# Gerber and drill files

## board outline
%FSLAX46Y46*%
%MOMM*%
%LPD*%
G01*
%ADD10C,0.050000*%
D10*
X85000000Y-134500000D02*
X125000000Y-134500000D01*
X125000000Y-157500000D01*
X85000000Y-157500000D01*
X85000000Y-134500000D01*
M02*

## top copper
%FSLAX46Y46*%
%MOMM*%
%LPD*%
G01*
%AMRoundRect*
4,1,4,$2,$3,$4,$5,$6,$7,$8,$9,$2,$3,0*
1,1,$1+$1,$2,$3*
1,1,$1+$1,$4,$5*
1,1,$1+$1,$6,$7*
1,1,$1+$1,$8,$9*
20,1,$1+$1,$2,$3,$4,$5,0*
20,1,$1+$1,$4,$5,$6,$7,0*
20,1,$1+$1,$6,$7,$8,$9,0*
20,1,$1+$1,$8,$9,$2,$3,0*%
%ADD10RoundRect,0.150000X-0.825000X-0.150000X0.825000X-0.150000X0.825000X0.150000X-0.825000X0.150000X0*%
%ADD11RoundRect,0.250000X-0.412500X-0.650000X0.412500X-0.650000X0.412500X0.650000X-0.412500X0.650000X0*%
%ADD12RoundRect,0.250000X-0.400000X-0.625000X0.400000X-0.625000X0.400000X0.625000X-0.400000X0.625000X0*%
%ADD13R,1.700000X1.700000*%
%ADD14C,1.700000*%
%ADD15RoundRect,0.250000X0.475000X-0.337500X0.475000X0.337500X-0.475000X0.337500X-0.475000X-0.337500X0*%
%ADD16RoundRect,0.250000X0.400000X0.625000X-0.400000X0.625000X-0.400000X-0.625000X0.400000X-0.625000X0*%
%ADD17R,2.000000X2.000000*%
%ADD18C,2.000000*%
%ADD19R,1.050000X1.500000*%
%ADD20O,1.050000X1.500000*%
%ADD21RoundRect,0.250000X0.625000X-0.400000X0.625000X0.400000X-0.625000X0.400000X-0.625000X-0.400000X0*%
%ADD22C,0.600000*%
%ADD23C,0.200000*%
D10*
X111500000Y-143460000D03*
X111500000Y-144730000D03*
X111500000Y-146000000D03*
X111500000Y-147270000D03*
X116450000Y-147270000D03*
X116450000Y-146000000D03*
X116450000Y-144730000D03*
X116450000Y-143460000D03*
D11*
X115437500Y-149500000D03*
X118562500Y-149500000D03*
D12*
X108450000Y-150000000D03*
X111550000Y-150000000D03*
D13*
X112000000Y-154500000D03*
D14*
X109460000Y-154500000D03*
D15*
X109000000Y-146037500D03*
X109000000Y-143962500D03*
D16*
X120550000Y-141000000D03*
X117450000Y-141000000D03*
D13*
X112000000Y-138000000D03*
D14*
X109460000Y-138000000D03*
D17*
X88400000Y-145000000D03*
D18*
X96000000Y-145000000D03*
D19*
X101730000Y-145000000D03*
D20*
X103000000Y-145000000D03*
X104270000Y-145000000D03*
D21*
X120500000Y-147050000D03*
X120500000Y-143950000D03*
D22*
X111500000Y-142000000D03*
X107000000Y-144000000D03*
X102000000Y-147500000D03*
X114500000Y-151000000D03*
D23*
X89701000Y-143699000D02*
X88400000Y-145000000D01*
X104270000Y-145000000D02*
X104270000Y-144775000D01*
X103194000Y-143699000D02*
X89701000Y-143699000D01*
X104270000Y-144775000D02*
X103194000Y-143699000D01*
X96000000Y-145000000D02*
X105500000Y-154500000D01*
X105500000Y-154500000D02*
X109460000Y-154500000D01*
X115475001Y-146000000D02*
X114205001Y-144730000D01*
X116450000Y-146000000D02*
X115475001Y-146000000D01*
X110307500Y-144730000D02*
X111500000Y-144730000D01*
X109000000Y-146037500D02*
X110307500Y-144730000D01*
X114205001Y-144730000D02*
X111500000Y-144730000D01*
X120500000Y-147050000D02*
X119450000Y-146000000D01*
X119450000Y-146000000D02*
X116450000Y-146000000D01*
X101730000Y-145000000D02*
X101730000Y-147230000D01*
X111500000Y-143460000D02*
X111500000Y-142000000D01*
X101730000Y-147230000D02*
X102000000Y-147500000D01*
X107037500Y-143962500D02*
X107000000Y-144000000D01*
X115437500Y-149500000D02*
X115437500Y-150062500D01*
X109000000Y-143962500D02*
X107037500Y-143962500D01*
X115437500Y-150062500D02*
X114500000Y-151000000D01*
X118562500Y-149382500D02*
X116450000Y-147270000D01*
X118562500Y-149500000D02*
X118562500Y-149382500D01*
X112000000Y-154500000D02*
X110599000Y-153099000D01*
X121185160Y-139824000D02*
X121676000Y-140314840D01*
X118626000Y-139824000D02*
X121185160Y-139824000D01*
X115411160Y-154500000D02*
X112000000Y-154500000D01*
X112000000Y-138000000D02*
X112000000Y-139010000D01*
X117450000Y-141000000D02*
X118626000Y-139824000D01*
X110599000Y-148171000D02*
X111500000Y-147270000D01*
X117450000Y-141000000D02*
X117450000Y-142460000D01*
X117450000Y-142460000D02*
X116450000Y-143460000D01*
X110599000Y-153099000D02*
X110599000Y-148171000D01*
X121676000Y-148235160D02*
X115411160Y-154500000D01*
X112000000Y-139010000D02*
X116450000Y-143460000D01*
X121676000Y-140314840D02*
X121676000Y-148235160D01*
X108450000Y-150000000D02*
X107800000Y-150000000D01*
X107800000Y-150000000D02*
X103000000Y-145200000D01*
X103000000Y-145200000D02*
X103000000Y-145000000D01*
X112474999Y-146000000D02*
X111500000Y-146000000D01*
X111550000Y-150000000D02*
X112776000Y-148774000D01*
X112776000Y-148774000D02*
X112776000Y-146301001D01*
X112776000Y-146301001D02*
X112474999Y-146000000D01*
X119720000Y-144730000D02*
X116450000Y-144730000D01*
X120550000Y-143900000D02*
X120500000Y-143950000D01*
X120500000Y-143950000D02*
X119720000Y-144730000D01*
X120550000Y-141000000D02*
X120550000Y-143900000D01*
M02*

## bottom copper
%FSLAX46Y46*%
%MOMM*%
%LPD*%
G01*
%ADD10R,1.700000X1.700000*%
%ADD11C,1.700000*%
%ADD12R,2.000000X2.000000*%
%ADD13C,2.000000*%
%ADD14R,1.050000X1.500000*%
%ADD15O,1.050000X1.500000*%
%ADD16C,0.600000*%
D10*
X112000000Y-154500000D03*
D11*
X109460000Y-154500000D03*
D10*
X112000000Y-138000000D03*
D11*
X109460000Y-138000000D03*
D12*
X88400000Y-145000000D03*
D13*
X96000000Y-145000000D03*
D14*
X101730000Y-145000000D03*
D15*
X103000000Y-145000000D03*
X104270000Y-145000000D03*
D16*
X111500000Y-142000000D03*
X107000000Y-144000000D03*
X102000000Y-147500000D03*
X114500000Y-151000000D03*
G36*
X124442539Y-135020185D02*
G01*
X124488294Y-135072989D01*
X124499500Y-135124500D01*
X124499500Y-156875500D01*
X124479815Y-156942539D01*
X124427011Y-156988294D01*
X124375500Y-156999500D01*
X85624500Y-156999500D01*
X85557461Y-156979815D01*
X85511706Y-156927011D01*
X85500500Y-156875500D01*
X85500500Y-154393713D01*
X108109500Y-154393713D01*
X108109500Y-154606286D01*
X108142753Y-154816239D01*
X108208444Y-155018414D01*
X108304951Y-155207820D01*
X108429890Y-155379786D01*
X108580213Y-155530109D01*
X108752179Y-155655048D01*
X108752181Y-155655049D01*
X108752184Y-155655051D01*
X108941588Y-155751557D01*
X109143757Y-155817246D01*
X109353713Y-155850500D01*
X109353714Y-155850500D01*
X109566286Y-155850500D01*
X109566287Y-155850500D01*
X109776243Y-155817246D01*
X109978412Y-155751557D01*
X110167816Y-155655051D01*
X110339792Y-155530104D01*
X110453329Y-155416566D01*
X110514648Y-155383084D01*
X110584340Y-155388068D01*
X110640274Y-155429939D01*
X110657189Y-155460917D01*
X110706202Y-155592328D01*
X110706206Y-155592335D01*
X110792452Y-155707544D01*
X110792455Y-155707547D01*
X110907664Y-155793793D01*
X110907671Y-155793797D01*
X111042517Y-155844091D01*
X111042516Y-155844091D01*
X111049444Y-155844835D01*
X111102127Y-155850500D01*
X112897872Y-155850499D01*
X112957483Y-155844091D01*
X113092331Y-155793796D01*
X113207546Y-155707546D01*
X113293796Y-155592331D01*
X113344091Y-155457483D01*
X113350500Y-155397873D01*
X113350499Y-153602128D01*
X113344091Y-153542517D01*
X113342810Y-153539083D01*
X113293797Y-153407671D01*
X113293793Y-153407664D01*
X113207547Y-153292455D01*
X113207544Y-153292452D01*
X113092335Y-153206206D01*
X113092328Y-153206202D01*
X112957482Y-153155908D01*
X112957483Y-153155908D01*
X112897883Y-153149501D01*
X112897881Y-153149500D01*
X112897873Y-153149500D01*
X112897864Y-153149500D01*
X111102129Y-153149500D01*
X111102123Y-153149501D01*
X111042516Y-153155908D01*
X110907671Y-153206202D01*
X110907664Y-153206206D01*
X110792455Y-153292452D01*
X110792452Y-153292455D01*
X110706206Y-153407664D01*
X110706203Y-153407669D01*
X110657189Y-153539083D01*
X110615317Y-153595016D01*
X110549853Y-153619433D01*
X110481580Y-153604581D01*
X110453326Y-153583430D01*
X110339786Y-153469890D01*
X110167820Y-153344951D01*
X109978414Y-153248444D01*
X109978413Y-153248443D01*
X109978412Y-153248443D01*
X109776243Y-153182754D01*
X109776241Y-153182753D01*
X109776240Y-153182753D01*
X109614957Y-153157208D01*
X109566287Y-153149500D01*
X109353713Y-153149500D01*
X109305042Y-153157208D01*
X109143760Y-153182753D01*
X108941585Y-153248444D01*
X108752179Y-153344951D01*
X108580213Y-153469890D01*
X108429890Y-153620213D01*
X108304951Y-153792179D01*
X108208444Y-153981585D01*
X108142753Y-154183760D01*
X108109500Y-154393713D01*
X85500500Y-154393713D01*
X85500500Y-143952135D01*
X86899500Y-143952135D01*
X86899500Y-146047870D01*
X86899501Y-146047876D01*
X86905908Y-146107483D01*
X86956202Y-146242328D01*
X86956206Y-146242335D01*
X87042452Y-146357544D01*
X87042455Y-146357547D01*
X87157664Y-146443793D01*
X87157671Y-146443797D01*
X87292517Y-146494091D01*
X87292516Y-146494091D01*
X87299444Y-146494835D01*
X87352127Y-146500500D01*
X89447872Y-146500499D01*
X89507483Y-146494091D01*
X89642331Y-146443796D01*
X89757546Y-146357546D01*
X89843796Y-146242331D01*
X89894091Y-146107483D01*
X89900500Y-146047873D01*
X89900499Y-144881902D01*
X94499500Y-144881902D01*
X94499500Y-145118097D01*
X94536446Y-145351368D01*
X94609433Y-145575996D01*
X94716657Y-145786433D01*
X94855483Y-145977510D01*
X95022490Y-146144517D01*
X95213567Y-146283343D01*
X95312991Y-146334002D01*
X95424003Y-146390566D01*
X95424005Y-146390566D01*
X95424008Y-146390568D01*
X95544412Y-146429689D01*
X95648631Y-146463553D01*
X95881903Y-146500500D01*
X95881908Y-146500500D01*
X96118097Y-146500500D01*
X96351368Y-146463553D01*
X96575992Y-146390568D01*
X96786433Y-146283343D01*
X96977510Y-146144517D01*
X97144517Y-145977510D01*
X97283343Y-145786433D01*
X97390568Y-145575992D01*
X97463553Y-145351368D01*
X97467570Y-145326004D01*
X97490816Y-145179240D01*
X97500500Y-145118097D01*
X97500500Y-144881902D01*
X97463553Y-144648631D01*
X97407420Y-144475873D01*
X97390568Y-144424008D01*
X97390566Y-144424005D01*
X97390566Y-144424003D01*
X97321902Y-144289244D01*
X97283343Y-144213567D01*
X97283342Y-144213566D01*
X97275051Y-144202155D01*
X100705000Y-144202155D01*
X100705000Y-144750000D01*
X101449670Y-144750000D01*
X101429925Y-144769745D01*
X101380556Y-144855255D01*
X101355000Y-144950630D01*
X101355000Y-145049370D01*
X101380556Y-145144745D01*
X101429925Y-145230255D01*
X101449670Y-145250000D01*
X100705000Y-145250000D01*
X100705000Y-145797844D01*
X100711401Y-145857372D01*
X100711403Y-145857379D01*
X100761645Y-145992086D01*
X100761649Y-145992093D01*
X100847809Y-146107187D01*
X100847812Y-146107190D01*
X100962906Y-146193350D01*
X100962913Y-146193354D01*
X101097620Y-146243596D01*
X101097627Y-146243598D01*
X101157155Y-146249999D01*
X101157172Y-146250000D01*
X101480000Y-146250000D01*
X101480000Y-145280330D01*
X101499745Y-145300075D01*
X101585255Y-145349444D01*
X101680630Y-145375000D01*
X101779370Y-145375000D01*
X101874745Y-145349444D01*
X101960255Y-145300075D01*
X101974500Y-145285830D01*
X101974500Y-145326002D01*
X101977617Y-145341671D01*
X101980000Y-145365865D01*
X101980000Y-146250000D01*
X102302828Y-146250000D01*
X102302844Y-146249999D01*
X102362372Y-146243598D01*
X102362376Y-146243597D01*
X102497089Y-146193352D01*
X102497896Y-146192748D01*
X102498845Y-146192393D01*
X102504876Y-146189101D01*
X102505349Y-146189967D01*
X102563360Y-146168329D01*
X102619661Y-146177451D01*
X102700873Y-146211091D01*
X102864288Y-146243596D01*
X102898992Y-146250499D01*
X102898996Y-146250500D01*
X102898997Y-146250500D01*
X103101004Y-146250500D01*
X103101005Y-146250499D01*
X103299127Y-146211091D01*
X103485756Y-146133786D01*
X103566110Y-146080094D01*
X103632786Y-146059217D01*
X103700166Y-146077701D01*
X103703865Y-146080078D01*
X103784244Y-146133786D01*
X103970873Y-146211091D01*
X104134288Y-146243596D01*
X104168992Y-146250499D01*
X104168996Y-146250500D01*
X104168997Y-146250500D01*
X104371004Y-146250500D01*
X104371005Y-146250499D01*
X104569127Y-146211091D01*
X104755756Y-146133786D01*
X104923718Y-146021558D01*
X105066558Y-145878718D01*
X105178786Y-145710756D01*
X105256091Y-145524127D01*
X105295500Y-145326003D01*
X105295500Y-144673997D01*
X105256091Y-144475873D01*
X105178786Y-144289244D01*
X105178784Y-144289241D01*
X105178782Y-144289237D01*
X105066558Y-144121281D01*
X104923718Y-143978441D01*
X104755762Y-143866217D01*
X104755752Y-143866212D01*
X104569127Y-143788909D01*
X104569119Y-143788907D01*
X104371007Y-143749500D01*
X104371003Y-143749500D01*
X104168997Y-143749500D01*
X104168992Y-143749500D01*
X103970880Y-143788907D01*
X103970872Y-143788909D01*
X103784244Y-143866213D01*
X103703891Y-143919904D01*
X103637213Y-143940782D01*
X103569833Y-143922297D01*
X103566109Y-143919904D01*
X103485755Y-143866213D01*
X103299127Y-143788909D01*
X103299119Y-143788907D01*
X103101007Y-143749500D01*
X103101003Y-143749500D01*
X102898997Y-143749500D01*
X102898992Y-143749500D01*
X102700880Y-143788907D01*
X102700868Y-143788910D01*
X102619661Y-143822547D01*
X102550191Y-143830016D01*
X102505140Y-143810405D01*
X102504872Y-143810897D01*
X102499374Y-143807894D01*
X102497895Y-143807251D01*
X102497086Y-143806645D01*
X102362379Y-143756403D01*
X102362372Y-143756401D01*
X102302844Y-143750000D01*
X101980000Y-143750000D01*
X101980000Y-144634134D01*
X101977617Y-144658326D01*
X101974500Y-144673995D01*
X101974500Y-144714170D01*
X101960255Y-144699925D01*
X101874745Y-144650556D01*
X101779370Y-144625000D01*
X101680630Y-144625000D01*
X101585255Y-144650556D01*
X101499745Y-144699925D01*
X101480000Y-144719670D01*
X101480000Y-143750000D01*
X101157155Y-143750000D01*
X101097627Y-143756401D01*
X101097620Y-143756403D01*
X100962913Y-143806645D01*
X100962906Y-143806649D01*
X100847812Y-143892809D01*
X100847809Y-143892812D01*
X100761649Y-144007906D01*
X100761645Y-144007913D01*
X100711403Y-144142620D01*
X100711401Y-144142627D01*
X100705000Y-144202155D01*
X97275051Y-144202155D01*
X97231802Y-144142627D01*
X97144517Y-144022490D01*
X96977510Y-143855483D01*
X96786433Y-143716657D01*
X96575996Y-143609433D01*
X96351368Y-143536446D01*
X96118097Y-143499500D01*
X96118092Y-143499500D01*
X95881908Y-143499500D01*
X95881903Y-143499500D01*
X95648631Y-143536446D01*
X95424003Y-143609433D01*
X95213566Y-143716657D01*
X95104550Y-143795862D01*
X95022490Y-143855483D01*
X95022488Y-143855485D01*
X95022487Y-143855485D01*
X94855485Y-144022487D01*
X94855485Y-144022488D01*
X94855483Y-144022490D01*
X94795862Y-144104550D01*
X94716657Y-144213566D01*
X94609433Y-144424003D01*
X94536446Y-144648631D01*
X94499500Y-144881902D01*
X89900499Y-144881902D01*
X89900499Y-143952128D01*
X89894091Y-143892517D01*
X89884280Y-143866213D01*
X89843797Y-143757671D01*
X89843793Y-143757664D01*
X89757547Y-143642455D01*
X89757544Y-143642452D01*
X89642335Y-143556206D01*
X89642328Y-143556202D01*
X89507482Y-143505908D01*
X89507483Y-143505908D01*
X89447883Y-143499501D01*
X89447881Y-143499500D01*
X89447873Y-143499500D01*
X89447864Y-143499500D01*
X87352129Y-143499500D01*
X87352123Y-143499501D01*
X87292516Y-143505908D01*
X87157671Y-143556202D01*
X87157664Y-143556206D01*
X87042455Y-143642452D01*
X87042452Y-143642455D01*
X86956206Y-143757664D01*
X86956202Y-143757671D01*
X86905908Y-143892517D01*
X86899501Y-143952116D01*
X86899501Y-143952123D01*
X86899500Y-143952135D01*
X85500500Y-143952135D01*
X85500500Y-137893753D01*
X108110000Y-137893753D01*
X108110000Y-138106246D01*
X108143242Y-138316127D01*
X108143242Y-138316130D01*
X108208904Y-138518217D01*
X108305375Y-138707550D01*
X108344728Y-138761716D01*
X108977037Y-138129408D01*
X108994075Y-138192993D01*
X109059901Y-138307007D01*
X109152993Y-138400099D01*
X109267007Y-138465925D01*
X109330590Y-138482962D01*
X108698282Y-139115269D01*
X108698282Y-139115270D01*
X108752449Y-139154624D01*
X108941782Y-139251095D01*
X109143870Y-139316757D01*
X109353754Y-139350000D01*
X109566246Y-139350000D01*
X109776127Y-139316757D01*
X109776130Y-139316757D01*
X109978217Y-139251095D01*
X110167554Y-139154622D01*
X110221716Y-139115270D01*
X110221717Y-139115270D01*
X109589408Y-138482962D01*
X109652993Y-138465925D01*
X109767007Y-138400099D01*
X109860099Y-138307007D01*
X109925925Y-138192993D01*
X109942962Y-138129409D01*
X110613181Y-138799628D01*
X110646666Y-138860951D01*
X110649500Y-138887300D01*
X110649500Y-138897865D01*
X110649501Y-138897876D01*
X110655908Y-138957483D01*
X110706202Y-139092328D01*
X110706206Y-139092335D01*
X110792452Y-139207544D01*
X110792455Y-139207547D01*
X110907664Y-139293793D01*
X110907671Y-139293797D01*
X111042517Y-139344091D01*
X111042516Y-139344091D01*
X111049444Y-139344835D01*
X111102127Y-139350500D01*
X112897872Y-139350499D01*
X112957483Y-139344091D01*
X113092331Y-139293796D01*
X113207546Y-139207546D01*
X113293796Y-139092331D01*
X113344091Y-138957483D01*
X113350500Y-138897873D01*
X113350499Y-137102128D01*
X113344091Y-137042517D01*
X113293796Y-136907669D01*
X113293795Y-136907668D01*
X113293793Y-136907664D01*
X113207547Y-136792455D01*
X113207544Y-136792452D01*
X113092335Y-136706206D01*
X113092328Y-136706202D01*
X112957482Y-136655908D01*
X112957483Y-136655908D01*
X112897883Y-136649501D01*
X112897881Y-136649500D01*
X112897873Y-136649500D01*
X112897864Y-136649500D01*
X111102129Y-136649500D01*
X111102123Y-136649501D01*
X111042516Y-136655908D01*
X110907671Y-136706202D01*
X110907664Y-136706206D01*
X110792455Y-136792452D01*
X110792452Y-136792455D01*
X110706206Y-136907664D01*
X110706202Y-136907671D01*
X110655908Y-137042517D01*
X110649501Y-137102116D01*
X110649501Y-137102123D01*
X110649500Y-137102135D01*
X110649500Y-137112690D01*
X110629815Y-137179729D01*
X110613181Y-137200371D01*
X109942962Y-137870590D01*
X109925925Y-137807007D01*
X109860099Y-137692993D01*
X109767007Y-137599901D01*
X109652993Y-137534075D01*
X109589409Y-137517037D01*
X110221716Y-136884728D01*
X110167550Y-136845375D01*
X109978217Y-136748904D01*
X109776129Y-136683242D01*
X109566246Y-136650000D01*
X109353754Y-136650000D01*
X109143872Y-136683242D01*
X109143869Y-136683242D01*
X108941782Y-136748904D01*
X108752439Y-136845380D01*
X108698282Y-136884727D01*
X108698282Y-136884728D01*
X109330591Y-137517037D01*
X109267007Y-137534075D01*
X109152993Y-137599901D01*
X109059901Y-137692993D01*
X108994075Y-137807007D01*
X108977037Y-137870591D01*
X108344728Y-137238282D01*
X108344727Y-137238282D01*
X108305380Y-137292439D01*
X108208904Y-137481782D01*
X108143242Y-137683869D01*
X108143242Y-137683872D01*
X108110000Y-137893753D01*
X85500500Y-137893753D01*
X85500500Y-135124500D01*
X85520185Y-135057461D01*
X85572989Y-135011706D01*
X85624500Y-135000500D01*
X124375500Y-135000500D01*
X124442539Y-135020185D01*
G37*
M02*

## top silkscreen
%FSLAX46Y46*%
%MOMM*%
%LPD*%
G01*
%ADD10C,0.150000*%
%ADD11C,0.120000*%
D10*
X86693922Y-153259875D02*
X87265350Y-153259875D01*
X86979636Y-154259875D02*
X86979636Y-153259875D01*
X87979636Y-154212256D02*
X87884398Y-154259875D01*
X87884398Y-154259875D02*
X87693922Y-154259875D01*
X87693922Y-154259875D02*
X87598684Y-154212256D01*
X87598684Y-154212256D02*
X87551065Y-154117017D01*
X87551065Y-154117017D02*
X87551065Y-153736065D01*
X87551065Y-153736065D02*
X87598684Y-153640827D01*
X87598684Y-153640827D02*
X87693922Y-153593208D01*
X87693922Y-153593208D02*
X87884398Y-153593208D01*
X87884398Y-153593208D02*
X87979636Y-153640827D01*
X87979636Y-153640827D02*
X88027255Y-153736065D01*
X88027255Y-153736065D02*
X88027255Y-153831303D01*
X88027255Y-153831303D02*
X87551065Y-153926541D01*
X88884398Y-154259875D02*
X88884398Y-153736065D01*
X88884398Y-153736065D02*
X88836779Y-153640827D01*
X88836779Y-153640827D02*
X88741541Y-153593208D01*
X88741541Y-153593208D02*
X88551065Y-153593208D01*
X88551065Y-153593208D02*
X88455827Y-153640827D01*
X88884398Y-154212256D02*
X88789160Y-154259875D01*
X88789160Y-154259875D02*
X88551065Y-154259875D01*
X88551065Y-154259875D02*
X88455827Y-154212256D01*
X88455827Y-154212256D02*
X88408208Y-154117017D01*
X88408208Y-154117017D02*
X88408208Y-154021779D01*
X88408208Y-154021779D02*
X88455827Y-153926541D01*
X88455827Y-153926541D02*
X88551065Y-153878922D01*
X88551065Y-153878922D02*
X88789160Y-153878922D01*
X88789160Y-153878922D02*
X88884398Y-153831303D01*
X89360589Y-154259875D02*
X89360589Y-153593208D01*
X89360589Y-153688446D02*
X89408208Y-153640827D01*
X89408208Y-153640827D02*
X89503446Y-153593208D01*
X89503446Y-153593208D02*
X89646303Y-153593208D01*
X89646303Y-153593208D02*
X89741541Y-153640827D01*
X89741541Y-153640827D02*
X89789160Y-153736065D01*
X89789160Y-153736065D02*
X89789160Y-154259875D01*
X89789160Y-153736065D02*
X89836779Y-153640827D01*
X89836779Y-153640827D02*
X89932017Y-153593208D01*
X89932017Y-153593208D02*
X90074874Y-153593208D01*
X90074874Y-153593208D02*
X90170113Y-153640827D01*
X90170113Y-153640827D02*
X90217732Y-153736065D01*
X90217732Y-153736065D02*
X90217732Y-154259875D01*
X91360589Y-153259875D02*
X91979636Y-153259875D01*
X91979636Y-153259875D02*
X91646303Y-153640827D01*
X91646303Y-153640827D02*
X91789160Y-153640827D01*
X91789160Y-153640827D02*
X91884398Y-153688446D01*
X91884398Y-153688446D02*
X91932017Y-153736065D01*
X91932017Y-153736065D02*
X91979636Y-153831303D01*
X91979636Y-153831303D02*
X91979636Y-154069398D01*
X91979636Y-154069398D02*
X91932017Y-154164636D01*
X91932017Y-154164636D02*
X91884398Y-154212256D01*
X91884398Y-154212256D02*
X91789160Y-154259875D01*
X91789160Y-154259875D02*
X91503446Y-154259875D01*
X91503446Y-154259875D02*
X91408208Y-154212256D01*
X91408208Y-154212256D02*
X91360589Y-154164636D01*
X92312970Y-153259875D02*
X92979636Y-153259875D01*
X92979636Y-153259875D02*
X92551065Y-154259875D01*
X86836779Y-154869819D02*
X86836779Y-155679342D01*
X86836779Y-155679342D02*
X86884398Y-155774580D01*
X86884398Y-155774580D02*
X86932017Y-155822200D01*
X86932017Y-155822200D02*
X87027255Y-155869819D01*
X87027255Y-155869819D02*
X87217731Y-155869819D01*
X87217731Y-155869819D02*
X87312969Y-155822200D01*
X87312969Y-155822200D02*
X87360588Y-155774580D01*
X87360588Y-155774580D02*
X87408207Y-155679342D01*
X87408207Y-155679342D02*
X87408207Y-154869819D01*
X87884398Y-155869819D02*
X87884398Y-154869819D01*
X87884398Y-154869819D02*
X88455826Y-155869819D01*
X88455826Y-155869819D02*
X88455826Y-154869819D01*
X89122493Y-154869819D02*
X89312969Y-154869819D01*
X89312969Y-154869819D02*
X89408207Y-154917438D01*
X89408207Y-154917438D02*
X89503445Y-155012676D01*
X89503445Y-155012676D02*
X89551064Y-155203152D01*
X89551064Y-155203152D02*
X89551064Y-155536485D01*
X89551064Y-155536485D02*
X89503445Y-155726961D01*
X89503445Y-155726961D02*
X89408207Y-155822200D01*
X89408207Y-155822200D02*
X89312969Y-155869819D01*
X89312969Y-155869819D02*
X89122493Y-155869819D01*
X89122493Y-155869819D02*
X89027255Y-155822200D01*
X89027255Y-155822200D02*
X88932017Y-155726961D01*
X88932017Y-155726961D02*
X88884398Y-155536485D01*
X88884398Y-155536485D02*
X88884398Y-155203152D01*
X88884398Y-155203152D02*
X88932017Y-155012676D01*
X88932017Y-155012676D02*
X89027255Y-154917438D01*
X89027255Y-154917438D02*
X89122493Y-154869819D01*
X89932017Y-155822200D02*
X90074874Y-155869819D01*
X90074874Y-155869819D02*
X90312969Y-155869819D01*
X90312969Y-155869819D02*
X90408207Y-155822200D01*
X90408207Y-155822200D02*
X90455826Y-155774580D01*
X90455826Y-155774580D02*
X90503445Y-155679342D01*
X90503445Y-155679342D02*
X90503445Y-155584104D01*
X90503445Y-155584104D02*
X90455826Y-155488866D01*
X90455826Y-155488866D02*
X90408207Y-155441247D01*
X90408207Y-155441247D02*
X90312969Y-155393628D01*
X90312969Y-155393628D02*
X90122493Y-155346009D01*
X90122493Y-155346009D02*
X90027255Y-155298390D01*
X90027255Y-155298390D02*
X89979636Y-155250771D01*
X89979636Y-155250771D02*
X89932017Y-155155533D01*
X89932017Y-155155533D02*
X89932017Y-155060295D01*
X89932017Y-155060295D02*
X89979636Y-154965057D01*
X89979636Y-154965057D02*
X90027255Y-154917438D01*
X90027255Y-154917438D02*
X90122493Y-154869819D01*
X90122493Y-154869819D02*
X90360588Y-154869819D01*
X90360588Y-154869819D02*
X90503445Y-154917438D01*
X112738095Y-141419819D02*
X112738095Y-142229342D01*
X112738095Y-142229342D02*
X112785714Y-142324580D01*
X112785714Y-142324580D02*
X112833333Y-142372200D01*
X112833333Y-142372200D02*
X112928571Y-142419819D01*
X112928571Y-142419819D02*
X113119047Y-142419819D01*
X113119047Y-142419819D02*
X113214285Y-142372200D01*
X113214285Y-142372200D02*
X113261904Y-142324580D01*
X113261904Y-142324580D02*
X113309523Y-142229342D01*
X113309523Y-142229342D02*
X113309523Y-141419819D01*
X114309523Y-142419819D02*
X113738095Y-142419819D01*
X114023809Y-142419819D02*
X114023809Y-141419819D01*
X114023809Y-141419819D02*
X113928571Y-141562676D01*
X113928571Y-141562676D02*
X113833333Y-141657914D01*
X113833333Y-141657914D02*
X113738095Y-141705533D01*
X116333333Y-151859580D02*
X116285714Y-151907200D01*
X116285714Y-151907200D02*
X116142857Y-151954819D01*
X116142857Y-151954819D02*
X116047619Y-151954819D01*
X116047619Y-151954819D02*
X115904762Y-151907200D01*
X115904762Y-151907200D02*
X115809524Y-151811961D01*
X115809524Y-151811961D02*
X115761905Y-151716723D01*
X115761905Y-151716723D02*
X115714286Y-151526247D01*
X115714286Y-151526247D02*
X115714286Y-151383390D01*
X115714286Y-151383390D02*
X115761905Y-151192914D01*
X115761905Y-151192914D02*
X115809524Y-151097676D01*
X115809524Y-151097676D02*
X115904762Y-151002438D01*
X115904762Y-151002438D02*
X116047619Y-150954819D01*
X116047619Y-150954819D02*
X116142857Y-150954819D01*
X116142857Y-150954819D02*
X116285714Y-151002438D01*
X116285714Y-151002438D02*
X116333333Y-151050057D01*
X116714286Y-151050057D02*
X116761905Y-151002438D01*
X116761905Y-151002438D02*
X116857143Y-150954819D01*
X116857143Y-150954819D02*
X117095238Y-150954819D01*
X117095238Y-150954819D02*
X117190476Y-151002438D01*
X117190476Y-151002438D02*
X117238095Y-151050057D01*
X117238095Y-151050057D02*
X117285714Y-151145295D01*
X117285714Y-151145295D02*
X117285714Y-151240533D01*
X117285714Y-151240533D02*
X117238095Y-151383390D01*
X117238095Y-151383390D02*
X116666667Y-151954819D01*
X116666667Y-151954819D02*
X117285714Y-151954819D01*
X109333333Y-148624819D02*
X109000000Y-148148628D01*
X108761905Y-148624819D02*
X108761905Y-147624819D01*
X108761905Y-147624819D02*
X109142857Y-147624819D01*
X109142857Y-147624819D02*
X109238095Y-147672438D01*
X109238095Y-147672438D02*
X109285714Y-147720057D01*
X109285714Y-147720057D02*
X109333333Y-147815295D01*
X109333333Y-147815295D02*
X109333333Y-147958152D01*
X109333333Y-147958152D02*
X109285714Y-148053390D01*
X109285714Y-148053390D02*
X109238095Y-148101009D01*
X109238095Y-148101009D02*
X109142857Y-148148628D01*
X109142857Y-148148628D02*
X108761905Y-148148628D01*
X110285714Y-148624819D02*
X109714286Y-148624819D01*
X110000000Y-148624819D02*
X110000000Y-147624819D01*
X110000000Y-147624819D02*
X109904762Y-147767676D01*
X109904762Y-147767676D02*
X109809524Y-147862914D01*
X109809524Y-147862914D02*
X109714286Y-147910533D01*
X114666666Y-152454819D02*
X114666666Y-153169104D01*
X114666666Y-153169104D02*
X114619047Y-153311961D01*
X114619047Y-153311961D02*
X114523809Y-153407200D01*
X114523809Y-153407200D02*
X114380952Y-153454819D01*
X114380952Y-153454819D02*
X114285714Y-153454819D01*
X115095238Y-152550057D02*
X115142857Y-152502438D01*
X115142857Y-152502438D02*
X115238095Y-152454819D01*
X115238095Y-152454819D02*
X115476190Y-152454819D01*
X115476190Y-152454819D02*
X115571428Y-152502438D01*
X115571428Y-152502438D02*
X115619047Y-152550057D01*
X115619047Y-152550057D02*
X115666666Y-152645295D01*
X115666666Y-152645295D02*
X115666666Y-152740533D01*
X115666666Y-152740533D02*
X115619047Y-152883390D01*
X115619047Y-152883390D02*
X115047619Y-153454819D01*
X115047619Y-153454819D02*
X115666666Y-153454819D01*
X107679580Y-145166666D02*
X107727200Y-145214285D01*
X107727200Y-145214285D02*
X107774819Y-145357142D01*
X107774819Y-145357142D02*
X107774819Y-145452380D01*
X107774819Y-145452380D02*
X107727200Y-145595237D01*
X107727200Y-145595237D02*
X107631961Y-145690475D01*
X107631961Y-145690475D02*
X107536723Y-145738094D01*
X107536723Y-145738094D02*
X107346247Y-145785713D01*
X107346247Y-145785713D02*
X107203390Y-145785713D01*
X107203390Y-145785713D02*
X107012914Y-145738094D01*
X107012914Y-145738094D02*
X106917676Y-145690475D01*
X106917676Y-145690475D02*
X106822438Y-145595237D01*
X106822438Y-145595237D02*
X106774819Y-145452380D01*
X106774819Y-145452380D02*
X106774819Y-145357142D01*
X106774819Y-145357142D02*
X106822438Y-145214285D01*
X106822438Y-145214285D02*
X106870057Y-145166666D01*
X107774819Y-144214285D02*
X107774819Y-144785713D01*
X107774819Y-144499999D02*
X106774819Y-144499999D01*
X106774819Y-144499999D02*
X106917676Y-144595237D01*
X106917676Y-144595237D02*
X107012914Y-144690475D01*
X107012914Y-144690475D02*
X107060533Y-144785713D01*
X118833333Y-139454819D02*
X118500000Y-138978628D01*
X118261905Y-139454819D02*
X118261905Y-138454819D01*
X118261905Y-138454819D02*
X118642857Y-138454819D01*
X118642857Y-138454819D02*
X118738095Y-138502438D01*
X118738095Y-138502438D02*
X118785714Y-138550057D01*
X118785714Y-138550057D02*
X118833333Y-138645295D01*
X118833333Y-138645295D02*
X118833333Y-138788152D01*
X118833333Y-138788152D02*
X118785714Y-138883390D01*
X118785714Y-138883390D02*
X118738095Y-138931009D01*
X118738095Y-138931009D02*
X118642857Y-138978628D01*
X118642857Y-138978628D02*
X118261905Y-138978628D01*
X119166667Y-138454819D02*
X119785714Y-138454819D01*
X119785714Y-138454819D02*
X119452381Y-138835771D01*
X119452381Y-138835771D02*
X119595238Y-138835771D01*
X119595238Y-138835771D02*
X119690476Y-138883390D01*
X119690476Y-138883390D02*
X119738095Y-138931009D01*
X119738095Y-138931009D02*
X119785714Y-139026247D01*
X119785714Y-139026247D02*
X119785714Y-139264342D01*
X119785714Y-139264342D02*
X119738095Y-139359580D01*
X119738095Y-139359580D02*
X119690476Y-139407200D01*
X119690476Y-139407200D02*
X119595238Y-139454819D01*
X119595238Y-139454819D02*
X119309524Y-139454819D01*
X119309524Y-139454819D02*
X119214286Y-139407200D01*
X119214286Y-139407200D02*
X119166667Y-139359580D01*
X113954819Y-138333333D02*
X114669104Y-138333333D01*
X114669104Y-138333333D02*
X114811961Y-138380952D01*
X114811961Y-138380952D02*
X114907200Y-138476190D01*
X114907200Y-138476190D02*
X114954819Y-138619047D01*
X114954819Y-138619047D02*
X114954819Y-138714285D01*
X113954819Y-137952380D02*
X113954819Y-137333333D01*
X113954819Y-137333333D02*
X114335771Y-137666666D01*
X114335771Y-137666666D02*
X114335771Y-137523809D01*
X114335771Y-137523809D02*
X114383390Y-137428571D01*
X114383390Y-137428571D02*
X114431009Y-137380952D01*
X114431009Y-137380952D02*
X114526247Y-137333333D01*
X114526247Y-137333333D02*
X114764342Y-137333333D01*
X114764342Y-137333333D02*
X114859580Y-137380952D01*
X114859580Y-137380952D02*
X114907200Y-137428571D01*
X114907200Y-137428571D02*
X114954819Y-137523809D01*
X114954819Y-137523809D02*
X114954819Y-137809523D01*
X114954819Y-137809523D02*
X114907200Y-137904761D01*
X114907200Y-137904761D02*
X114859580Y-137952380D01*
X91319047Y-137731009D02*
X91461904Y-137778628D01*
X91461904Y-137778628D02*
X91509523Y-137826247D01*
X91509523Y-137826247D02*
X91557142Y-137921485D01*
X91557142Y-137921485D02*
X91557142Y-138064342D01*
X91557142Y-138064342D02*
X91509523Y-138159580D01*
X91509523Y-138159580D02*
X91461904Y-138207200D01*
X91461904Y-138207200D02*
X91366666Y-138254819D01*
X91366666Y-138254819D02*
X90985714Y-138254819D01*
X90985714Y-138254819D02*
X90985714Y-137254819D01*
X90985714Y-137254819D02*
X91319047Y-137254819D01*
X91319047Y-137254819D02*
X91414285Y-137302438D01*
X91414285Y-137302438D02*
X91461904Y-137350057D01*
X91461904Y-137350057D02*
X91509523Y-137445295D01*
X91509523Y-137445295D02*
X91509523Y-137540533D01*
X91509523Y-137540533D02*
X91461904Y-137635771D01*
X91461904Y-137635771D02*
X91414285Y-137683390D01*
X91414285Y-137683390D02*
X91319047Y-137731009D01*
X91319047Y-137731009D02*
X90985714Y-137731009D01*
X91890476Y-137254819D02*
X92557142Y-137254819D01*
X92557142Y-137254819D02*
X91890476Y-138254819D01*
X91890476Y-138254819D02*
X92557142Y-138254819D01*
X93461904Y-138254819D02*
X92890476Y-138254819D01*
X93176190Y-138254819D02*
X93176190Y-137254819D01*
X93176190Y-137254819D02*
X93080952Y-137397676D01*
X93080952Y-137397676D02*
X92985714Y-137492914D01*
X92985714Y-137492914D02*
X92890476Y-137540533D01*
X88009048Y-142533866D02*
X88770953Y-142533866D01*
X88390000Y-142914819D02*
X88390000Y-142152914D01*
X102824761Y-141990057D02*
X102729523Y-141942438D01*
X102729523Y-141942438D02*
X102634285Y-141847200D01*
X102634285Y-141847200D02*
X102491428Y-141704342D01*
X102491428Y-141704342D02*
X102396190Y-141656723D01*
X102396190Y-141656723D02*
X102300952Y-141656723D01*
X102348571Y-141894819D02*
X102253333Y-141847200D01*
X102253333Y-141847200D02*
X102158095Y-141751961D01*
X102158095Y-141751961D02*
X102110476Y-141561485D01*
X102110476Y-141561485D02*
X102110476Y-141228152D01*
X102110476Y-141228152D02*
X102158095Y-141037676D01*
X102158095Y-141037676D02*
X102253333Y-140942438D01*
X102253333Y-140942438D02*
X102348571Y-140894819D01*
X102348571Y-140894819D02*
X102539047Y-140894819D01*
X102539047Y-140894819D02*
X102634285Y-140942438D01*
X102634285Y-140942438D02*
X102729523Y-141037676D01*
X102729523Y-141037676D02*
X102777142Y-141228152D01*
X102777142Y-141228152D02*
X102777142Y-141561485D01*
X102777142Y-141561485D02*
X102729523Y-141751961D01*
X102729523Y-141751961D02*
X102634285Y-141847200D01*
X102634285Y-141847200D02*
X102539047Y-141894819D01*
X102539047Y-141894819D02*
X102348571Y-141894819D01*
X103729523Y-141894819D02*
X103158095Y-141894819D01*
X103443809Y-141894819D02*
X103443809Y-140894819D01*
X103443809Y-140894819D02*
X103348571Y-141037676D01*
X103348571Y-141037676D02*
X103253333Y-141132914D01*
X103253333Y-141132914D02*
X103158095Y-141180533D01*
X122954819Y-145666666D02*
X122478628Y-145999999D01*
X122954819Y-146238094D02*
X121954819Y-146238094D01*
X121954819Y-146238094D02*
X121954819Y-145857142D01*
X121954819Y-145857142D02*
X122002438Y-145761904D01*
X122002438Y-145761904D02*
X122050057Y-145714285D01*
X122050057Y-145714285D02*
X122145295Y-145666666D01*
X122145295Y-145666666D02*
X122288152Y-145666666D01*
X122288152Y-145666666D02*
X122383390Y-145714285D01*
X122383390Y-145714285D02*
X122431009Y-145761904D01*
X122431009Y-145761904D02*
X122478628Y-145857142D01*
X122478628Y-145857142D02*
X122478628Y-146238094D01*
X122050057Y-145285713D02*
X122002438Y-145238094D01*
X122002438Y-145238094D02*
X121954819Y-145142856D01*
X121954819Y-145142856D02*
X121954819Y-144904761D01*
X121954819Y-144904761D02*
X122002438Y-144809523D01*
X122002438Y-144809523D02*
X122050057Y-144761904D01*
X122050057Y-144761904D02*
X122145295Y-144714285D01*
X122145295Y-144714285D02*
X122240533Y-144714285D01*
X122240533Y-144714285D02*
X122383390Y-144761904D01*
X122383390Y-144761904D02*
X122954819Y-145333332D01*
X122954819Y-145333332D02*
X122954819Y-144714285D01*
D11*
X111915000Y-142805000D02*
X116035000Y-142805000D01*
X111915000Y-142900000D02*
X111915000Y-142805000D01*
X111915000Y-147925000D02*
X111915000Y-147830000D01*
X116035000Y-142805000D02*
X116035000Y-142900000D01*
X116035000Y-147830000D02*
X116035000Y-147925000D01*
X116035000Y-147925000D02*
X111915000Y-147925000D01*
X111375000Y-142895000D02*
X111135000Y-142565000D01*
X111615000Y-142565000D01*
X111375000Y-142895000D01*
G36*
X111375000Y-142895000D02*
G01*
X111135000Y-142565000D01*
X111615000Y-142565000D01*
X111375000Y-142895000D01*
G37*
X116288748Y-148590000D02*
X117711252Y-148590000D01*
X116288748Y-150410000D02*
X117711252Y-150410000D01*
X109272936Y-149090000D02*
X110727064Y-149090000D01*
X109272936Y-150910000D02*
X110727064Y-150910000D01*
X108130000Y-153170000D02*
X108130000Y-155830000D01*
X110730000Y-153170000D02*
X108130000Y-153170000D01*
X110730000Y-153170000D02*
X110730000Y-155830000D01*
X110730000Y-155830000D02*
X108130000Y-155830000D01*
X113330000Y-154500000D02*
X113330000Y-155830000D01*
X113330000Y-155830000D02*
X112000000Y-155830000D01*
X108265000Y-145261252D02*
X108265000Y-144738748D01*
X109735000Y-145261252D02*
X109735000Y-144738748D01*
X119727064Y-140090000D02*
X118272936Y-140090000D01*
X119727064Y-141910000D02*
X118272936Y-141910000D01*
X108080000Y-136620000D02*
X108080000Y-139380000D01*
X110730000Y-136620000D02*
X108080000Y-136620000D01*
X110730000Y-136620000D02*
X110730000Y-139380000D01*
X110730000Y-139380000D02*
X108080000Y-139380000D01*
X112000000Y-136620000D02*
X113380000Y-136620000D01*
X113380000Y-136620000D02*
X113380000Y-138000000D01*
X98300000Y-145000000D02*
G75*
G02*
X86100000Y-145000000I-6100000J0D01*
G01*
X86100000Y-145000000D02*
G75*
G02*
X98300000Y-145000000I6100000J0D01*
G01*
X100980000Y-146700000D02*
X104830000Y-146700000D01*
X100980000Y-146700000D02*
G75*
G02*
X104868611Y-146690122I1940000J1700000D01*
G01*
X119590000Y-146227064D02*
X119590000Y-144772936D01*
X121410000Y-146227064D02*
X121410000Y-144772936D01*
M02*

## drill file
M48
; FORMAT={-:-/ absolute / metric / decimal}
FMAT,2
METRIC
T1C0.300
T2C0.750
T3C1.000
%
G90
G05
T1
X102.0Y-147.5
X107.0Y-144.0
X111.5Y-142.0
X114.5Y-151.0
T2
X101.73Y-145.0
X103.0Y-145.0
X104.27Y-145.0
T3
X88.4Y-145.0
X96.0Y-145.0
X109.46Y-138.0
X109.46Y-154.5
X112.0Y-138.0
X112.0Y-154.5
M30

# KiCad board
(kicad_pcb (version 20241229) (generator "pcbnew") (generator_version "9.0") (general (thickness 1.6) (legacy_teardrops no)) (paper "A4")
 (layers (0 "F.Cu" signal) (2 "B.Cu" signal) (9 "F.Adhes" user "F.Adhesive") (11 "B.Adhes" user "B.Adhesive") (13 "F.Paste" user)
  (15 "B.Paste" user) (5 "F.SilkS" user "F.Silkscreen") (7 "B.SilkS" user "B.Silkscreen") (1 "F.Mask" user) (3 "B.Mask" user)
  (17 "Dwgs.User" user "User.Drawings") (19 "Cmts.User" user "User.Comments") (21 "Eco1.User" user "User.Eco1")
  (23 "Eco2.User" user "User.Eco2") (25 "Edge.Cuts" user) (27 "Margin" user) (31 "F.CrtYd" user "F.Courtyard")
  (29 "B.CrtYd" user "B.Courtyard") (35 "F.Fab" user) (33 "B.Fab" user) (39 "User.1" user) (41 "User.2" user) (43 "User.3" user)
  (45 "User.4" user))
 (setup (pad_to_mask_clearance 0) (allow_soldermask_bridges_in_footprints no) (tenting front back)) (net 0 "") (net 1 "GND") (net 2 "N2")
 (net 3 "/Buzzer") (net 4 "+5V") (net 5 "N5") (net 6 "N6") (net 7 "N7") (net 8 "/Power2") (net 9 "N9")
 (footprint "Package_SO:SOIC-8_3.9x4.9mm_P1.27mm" (layer "F.Cu") (at 113.975 145.365)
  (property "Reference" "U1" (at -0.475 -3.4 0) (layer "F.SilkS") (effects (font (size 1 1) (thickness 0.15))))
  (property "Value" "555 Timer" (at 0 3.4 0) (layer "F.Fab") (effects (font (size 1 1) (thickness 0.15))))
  (fp_line (start -2.06 -2.56) (end 2.06 -2.56) (stroke (width 0.12) (type solid)) (layer "F.SilkS"))
  (fp_line (start -2.06 -2.465) (end -2.06 -2.56) (stroke (width 0.12) (type solid)) (layer "F.SilkS"))
  (fp_line (start -2.06 2.56) (end -2.06 2.465) (stroke (width 0.12) (type solid)) (layer "F.SilkS"))
  (fp_line (start 2.06 -2.56) (end 2.06 -2.465) (stroke (width 0.12) (type solid)) (layer "F.SilkS"))
  (fp_line (start 2.06 2.465) (end 2.06 2.56) (stroke (width 0.12) (type solid)) (layer "F.SilkS"))
  (fp_line (start 2.06 2.56) (end -2.06 2.56) (stroke (width 0.12) (type solid)) (layer "F.SilkS"))
  (fp_poly (pts (xy -2.6 -2.47) (xy -2.84 -2.8) (xy -2.36 -2.8)) (stroke (width 0.12) (type solid)) (fill yes) (layer "F.SilkS"))
  (pad "1" smd roundrect (at -2.475 -1.905) (size 1.95 0.6) (layers "F.Cu" "F.Mask" "F.Paste") (roundrect_rratio 0.25) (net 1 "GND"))
  (pad "2" smd roundrect (at -2.475 -0.635) (size 1.95 0.6) (layers "F.Cu" "F.Mask" "F.Paste") (roundrect_rratio 0.25) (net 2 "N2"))
  (pad "3" smd roundrect (at -2.475 0.635) (size 1.95 0.6) (layers "F.Cu" "F.Mask" "F.Paste") (roundrect_rratio 0.25) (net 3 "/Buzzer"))
  (pad "4" smd roundrect (at -2.475 1.905) (size 1.95 0.6) (layers "F.Cu" "F.Mask" "F.Paste") (roundrect_rratio 0.25) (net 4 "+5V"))
  (pad "5" smd roundrect (at 2.475 1.905) (size 1.95 0.6) (layers "F.Cu" "F.Mask" "F.Paste") (roundrect_rratio 0.25) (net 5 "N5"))
  (pad "6" smd roundrect (at 2.475 0.635) (size 1.95 0.6) (layers "F.Cu" "F.Mask" "F.Paste") (roundrect_rratio 0.25) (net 2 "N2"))
  (pad "7" smd roundrect (at 2.475 -0.635) (size 1.95 0.6) (layers "F.Cu" "F.Mask" "F.Paste") (roundrect_rratio 0.25) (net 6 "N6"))
  (pad "8" smd roundrect (at 2.475 -1.905) (size 1.95 0.6) (layers "F.Cu" "F.Mask" "F.Paste") (roundrect_rratio 0.25) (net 4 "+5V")))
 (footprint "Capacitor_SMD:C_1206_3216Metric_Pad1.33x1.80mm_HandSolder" (layer "F.Cu") (at 117 149.5)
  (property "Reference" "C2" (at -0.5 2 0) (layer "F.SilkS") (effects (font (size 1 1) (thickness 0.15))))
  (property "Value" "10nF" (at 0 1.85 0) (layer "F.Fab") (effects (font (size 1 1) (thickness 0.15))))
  (fp_line (start -0.711252 -0.91) (end 0.711252 -0.91) (stroke (width 0.12) (type solid)) (layer "F.SilkS"))
  (fp_line (start -0.711252 0.91) (end 0.711252 0.91) (stroke (width 0.12) (type solid)) (layer "F.SilkS"))
  (pad "1" smd roundrect (at -1.5625 0) (size 1.325 1.8) (layers "F.Cu" "F.Mask" "F.Paste") (roundrect_rratio 0.188679) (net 1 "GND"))
  (pad "2" smd roundrect (at 1.5625 0) (size 1.325 1.8) (layers "F.Cu" "F.Mask" "F.Paste") (roundrect_rratio 0.188679) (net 5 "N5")))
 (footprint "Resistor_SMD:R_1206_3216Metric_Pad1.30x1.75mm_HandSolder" (layer "F.Cu") (at 110 150)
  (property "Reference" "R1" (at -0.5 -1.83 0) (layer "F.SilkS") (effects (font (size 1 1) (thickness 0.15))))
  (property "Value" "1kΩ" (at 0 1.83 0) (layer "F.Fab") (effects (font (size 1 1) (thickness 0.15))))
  (fp_line (start -0.727064 -0.91) (end 0.727064 -0.91) (stroke (width 0.12) (type solid)) (layer "F.SilkS"))
  (fp_line (start -0.727064 0.91) (end 0.727064 0.91) (stroke (width 0.12) (type solid)) (layer "F.SilkS"))
  (pad "1" smd roundrect (at -1.55 0) (size 1.3 1.75) (layers "F.Cu" "F.Mask" "F.Paste") (roundrect_rratio 0.192308) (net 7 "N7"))
  (pad "2" smd roundrect (at 1.55 0) (size 1.3 1.75) (layers "F.Cu" "F.Mask" "F.Paste") (roundrect_rratio 0.192308) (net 3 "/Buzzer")))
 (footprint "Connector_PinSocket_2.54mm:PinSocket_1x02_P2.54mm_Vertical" (layer "F.Cu") (at 112 154.5 -90)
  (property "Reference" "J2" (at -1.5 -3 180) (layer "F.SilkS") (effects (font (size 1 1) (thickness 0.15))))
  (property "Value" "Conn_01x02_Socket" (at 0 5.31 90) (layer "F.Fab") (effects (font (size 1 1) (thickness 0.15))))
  (fp_line (start -1.33 3.87) (end 1.33 3.87) (stroke (width 0.12) (type solid)) (layer "F.SilkS"))
  (fp_line (start -1.33 1.27) (end -1.33 3.87) (stroke (width 0.12) (type solid)) (layer "F.SilkS"))
  (fp_line (start -1.33 1.27) (end 1.33 1.27) (stroke (width 0.12) (type solid)) (layer "F.SilkS"))
  (fp_line (start 1.33 1.27) (end 1.33 3.87) (stroke (width 0.12) (type solid)) (layer "F.SilkS"))
  (fp_line (start 0 -1.33) (end 1.33 -1.33) (stroke (width 0.12) (type solid)) (layer "F.SilkS"))
  (fp_line (start 1.33 -1.33) (end 1.33 0) (stroke (width 0.12) (type solid)) (layer "F.SilkS"))
  (pad "1" thru_hole rect (at 0 0 270) (size 1.7 1.7) (drill 1) (layers "*.Cu" "*.Mask") (remove_unused_layers no) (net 4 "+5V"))
  (pad "2" thru_hole circle (at 0 2.54 270) (size 1.7 1.7) (drill 1) (layers "*.Cu" "*.Mask") (remove_unused_layers no) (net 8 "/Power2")))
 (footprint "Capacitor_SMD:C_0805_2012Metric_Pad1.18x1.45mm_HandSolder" (layer "F.Cu") (at 109 145 90)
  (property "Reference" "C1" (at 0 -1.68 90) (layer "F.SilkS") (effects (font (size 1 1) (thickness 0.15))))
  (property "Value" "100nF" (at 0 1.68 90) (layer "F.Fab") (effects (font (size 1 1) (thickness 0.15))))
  (fp_line (start -0.261252 -0.735) (end 0.261252 -0.735) (stroke (width 0.12) (type solid)) (layer "F.SilkS"))
  (fp_line (start -0.261252 0.735) (end 0.261252 0.735) (stroke (width 0.12) (type solid)) (layer "F.SilkS"))
  (pad "1" smd roundrect (at -1.0375 0 90) (size 1.175 1.45) (layers "F.Cu" "F.Mask" "F.Paste") (roundrect_rratio 0.212766) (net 2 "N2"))
  (pad "2" smd roundrect (at 1.0375 0 90) (size 1.175 1.45) (layers "F.Cu" "F.Mask" "F.Paste") (roundrect_rratio 0.212766) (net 1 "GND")))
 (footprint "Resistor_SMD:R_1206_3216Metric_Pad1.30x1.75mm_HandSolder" (layer "F.Cu") (at 119 141 180)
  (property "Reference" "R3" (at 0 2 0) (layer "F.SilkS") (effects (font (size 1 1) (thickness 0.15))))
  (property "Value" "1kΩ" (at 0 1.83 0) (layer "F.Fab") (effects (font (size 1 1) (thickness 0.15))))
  (fp_line (start -0.727064 0.91) (end 0.727064 0.91) (stroke (width 0.12) (type solid)) (layer "F.SilkS"))
  (fp_line (start -0.727064 -0.91) (end 0.727064 -0.91) (stroke (width 0.12) (type solid)) (layer "F.SilkS"))
  (pad "1" smd roundrect (at -1.55 0 180) (size 1.3 1.75) (layers "F.Cu" "F.Mask" "F.Paste") (roundrect_rratio 0.192308) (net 6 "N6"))
  (pad "2" smd roundrect (at 1.55 0 180) (size 1.3 1.75) (layers "F.Cu" "F.Mask" "F.Paste") (roundrect_rratio 0.192308) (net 4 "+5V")))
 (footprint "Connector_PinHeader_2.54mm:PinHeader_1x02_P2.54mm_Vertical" (layer "F.Cu") (at 112 138 -90)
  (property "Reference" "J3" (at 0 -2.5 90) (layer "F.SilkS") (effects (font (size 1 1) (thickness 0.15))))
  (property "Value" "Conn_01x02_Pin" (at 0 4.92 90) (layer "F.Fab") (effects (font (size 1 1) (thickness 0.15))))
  (fp_line (start -1.38 3.92) (end 1.38 3.92) (stroke (width 0.12) (type solid)) (layer "F.SilkS"))
  (fp_line (start -1.38 1.27) (end -1.38 3.92) (stroke (width 0.12) (type solid)) (layer "F.SilkS"))
  (fp_line (start -1.38 1.27) (end 1.38 1.27) (stroke (width 0.12) (type solid)) (layer "F.SilkS"))
  (fp_line (start 1.38 1.27) (end 1.38 3.92) (stroke (width 0.12) (type solid)) (layer "F.SilkS"))
  (fp_line (start -1.38 0) (end -1.38 -1.38) (stroke (width 0.12) (type solid)) (layer "F.SilkS"))
  (fp_line (start -1.38 -1.38) (end 0 -1.38) (stroke (width 0.12) (type solid)) (layer "F.SilkS"))
  (pad "1" thru_hole rect (at 0 0 270) (size 1.7 1.7) (drill 1) (layers "*.Cu" "*.Mask") (remove_unused_layers no) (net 4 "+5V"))
  (pad "2" thru_hole circle (at 0 2.54 270) (size 1.7 1.7) (drill 1) (layers "*.Cu" "*.Mask") (remove_unused_layers no) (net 1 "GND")))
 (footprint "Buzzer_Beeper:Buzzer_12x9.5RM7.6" (layer "F.Cu") (at 88.4 145)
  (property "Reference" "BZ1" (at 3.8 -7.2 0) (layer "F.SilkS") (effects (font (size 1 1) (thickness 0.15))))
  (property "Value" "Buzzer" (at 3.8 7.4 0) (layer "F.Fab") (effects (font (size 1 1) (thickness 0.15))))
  (fp_circle (center 3.8 0) (end 9.9 0) (stroke (width 0.12) (type solid)) (fill no) (layer "F.SilkS"))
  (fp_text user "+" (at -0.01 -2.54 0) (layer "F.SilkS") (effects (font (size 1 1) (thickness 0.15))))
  (pad "1" thru_hole rect (at 0 0) (size 2 2) (drill 1) (layers "*.Cu" "*.Mask") (remove_unused_layers no) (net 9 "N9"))
  (pad "2" thru_hole circle (at 7.6 0) (size 2 2) (drill 1) (layers "*.Cu" "*.Mask") (remove_unused_layers no) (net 8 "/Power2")))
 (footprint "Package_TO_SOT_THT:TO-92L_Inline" (layer "F.Cu") (at 101.73 145)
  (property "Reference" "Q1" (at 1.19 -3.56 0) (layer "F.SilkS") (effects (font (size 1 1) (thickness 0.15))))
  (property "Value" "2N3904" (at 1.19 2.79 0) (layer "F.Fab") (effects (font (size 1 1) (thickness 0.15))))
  (fp_line (start -0.75 1.7) (end 3.1 1.7) (stroke (width 0.12) (type solid)) (layer "F.SilkS"))
  (fp_arc (start -0.75 1.7) (mid 1.183448 -2.579449) (end 3.138611 1.690122) (stroke (width 0.12) (type solid)) (layer "F.SilkS"))
  (pad "1" thru_hole rect (at 0 0) (size 1.05 1.5) (drill 0.75) (layers "*.Cu" "*.Mask") (remove_unused_layers no) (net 1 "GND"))
  (pad "2" thru_hole oval (at 1.27 0) (size 1.05 1.5) (drill 0.75) (layers "*.Cu" "*.Mask") (remove_unused_layers no) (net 7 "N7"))
  (pad "3" thru_hole oval (at 2.54 0) (size 1.05 1.5) (drill 0.75) (layers "*.Cu" "*.Mask") (remove_unused_layers no) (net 9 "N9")))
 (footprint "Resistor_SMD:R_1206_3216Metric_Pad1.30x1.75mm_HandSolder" (layer "F.Cu") (at 120.5 145.5 90)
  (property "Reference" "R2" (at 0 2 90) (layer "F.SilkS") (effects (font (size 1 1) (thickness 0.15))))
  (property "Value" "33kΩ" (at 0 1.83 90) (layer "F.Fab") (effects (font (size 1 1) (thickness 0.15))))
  (fp_line (start -0.727064 -0.91) (end 0.727064 -0.91) (stroke (width 0.12) (type solid)) (layer "F.SilkS"))
  (fp_line (start -0.727064 0.91) (end 0.727064 0.91) (stroke (width 0.12) (type solid)) (layer "F.SilkS"))
  (pad "1" smd roundrect (at -1.55 0 90) (size 1.3 1.75) (layers "F.Cu" "F.Mask" "F.Paste") (roundrect_rratio 0.192308) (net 2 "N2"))
  (pad "2" smd roundrect (at 1.55 0 90) (size 1.3 1.75) (layers "F.Cu" "F.Mask" "F.Paste") (roundrect_rratio 0.192308) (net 6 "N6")))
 (gr_rect (start 85 134.5) (end 125 157.5) (stroke (width 0.05) (type default)) (fill no) (layer "Edge.Cuts"))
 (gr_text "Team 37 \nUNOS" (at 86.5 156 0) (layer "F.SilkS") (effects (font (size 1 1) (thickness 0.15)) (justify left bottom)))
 (segment (start 89.701 143.699) (end 88.4 145) (width 0.2) (layer "F.Cu") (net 9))
 (segment (start 104.27 145) (end 104.27 144.775) (width 0.2) (layer "F.Cu") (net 9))
 (segment (start 103.194 143.699) (end 89.701 143.699) (width 0.2) (layer "F.Cu") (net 9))
 (segment (start 104.27 144.775) (end 103.194 143.699) (width 0.2) (layer "F.Cu") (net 9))
 (segment (start 96 145) (end 105.5 154.5) (width 0.2) (layer "F.Cu") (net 8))
 (segment (start 105.5 154.5) (end 109.46 154.5) (width 0.2) (layer "F.Cu") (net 8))
 (segment (start 115.475001 146) (end 114.205001 144.73) (width 0.2) (layer "F.Cu") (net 2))
 (segment (start 116.45 146) (end 115.475001 146) (width 0.2) (layer "F.Cu") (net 2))
 (segment (start 110.3075 144.73) (end 111.5 144.73) (width 0.2) (layer "F.Cu") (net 2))
 (segment (start 109 146.0375) (end 110.3075 144.73) (width 0.2) (layer "F.Cu") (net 2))
 (segment (start 114.205001 144.73) (end 111.5 144.73) (width 0.2) (layer "F.Cu") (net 2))
 (segment (start 120.5 147.05) (end 119.45 146) (width 0.2) (layer "F.Cu") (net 2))
 (segment (start 119.45 146) (end 116.45 146) (width 0.2) (layer "F.Cu") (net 2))
 (segment (start 101.73 145) (end 101.73 147.23) (width 0.2) (layer "F.Cu") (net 1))
 (segment (start 111.5 143.46) (end 111.5 142) (width 0.2) (layer "F.Cu") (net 1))
 (segment (start 101.73 147.23) (end 102 147.5) (width 0.2) (layer "F.Cu") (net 1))
 (segment (start 107.0375 143.9625) (end 107 144) (width 0.2) (layer "F.Cu") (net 1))
 (segment (start 115.4375 149.5) (end 115.4375 150.0625) (width 0.2) (layer "F.Cu") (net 1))
 (segment (start 109 143.9625) (end 107.0375 143.9625) (width 0.2) (layer "F.Cu") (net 1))
 (segment (start 115.4375 150.0625) (end 114.5 151) (width 0.2) (layer "F.Cu") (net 1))
 (via (at 111.5 142) (size 0.6) (drill 0.3) (layers "F.Cu" "B.Cu") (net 1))
 (via (at 107 144) (size 0.6) (drill 0.3) (layers "F.Cu" "B.Cu") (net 1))
 (via (at 102 147.5) (size 0.6) (drill 0.3) (layers "F.Cu" "B.Cu") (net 1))
 (via (at 114.5 151) (size 0.6) (drill 0.3) (layers "F.Cu" "B.Cu") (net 1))
 (segment (start 118.5625 149.3825) (end 116.45 147.27) (width 0.2) (layer "F.Cu") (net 5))
 (segment (start 118.5625 149.5) (end 118.5625 149.3825) (width 0.2) (layer "F.Cu") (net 5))
 (segment (start 112 154.5) (end 110.599 153.099) (width 0.2) (layer "F.Cu") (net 4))
 (segment (start 121.18516 139.824) (end 121.676 140.31484) (width 0.2) (layer "F.Cu") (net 4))
 (segment (start 118.626 139.824) (end 121.18516 139.824) (width 0.2) (layer "F.Cu") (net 4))
 (segment (start 115.41116 154.5) (end 112 154.5) (width 0.2) (layer "F.Cu") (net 4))
 (segment (start 112 138) (end 112 139.01) (width 0.2) (layer "F.Cu") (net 4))
 (segment (start 117.45 141) (end 118.626 139.824) (width 0.2) (layer "F.Cu") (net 4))
 (segment (start 110.599 148.171) (end 111.5 147.27) (width 0.2) (layer "F.Cu") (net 4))
 (segment (start 117.45 141) (end 117.45 142.46) (width 0.2) (layer "F.Cu") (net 4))
 (segment (start 117.45 142.46) (end 116.45 143.46) (width 0.2) (layer "F.Cu") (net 4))
 (segment (start 110.599 153.099) (end 110.599 148.171) (width 0.2) (layer "F.Cu") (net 4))
 (segment (start 121.676 148.23516) (end 115.41116 154.5) (width 0.2) (layer "F.Cu") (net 4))
 (segment (start 112 139.01) (end 116.45 143.46) (width 0.2) (layer "F.Cu") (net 4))
 (segment (start 121.676 140.31484) (end 121.676 148.23516) (width 0.2) (layer "F.Cu") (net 4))
 (segment (start 108.45 150) (end 107.8 150) (width 0.2) (layer "F.Cu") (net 7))
 (segment (start 107.8 150) (end 103 145.2) (width 0.2) (layer "F.Cu") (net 7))
 (segment (start 103 145.2) (end 103 145) (width 0.2) (layer "F.Cu") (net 7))
 (segment (start 112.474999 146) (end 111.5 146) (width 0.2) (layer "F.Cu") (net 3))
 (segment (start 111.55 150) (end 112.776 148.774) (width 0.2) (layer "F.Cu") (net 3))
 (segment (start 112.776 148.774) (end 112.776 146.301001) (width 0.2) (layer "F.Cu") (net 3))
 (segment (start 112.776 146.301001) (end 112.474999 146) (width 0.2) (layer "F.Cu") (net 3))
 (segment (start 119.72 144.73) (end 116.45 144.73) (width 0.2) (layer "F.Cu") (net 6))
 (segment (start 120.55 143.9) (end 120.5 143.95) (width 0.2) (layer "F.Cu") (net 6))
 (segment (start 120.5 143.95) (end 119.72 144.73) (width 0.2) (layer "F.Cu") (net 6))
 (segment (start 120.55 141) (end 120.55 143.9) (width 0.2) (layer "F.Cu") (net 6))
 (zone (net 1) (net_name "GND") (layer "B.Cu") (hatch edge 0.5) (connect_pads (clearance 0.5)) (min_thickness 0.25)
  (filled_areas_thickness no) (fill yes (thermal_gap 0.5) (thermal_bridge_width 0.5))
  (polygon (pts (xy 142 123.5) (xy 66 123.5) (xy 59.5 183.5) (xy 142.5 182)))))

